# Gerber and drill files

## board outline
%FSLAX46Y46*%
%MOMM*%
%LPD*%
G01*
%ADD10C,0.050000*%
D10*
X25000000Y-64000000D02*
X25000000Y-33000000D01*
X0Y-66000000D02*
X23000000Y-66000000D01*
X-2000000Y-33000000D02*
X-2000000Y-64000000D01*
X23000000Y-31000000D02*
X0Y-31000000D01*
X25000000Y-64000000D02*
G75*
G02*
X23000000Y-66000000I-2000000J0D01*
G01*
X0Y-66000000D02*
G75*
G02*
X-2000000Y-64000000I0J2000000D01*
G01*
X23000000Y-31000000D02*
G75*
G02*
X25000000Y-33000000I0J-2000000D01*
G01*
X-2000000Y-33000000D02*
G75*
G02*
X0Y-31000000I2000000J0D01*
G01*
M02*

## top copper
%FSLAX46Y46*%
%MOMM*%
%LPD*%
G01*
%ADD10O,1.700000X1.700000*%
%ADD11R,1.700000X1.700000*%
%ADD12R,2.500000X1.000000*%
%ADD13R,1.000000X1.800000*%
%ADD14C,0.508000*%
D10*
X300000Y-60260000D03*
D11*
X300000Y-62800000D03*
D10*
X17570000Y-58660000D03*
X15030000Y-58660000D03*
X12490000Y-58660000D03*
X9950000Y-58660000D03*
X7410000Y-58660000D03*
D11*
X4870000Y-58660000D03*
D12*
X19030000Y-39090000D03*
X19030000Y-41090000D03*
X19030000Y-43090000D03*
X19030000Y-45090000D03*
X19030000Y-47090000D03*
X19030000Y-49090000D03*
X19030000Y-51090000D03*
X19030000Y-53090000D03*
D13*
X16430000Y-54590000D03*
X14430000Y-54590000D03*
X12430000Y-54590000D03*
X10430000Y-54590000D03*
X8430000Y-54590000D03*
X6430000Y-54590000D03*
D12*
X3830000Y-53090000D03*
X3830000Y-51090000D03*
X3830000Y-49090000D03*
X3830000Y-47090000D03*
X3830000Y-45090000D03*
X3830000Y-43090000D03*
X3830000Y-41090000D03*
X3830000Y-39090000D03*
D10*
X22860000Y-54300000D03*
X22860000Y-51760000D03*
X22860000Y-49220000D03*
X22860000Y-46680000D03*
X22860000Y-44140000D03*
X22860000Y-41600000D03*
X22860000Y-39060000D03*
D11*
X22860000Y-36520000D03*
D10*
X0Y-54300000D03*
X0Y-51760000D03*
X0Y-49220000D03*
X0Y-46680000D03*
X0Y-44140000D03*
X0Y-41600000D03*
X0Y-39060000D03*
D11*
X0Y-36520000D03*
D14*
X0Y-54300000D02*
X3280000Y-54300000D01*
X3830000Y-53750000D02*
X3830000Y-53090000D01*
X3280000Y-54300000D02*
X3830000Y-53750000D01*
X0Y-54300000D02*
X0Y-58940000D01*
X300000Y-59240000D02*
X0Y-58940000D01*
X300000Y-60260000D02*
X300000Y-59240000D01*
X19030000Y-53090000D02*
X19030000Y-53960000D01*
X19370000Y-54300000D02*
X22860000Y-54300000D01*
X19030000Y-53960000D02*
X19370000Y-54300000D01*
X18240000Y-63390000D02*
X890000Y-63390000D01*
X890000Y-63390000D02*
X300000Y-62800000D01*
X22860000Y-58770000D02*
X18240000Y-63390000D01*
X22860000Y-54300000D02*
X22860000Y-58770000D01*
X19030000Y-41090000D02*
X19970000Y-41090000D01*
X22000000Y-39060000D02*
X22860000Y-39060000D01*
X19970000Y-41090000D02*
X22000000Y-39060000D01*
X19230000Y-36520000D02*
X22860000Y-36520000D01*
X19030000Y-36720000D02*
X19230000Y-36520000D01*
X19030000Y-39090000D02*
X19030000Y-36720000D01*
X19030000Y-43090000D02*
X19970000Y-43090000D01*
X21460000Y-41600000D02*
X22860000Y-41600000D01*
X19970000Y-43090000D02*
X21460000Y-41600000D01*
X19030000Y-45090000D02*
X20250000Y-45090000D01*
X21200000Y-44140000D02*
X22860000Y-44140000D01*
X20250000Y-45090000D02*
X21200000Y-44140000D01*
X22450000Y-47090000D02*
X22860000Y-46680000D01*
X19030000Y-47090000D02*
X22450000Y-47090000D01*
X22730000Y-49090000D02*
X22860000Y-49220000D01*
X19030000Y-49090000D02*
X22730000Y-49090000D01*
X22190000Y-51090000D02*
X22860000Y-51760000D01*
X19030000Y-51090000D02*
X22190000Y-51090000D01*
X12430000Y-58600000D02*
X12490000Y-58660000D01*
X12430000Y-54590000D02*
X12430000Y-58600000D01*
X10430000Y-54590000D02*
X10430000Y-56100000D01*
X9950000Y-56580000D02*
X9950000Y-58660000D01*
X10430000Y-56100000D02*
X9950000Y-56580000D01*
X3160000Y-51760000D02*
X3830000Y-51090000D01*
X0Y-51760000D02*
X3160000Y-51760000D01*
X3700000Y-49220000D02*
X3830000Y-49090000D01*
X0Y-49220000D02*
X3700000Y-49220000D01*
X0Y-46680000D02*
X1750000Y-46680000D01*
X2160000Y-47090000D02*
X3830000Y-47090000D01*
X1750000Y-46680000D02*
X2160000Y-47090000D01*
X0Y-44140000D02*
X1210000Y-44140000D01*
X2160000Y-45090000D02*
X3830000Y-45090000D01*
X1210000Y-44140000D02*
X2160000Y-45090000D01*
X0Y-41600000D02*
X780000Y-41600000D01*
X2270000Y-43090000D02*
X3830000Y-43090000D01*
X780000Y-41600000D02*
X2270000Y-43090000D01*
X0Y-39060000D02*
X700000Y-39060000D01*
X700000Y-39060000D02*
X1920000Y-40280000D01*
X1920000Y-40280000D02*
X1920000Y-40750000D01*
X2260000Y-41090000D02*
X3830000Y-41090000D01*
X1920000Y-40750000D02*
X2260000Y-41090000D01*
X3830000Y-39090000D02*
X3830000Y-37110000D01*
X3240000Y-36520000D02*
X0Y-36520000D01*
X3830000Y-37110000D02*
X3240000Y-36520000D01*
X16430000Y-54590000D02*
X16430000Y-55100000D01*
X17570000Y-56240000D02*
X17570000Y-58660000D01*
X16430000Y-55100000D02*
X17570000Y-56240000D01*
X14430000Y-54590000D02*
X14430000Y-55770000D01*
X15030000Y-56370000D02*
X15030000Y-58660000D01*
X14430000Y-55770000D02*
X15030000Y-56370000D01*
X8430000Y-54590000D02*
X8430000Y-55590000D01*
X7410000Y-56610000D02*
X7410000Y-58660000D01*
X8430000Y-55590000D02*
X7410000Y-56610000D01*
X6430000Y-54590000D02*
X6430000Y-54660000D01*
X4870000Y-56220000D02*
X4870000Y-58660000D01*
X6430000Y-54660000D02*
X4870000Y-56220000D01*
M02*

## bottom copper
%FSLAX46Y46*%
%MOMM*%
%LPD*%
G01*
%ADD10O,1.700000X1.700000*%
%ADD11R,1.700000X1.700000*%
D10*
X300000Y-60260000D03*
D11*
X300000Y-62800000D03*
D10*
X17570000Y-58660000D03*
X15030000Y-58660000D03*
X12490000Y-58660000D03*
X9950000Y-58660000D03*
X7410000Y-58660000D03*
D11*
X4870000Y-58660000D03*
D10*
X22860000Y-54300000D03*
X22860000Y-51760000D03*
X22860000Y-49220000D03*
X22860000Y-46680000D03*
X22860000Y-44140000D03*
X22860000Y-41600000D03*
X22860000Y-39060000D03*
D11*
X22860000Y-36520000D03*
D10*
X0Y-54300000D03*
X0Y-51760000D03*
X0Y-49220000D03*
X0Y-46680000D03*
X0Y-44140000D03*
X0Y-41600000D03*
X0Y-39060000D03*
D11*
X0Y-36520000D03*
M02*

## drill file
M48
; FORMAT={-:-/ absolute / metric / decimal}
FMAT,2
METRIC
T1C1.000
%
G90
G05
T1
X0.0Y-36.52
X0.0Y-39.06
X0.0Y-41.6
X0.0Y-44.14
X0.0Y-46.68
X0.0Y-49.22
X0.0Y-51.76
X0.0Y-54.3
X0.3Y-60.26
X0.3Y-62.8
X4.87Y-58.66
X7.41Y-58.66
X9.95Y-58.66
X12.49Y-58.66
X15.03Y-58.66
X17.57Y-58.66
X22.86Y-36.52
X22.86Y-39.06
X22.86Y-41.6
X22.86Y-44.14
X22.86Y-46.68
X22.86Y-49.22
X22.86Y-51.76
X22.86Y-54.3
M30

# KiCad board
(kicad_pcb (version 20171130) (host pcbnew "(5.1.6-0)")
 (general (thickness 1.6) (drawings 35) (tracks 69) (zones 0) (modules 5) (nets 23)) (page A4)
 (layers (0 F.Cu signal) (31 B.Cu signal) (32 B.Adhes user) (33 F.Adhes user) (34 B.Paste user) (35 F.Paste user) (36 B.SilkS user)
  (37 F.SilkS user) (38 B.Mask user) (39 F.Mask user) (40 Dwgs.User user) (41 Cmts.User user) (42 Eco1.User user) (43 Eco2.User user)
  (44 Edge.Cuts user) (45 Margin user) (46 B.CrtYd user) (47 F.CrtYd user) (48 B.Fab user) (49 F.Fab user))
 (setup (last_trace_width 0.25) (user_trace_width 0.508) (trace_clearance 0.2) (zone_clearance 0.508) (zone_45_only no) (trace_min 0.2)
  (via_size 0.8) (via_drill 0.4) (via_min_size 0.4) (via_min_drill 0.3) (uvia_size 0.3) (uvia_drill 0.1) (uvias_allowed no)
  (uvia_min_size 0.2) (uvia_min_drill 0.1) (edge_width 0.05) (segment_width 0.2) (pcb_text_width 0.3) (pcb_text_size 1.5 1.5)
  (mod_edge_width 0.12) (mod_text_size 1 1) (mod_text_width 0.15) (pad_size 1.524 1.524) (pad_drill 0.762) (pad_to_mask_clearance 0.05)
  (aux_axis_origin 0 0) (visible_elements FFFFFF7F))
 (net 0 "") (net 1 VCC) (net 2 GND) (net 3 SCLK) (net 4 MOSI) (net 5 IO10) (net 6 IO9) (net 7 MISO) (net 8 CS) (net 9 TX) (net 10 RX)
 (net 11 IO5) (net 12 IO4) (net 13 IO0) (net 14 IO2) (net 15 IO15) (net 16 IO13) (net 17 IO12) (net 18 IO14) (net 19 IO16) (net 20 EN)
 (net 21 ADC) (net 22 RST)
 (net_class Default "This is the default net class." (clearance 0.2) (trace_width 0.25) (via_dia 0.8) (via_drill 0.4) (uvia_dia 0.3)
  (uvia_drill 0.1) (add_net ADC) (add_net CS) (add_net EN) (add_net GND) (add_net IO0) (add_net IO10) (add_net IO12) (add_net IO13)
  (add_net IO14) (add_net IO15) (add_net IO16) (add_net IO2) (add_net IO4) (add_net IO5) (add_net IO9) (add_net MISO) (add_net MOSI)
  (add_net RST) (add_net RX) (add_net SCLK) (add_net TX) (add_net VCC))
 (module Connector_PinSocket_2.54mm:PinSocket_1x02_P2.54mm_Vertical (layer F.Cu) (at 0.3 62.8 180)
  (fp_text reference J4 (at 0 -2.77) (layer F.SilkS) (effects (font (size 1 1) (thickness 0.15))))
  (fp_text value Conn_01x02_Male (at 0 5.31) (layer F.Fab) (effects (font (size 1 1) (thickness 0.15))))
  (pad 2 thru_hole oval (at 0 2.54 180) (size 1.7 1.7) (drill 1) (layers *.Cu *.Mask) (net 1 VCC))
  (pad 1 thru_hole rect (at 0 0 180) (size 1.7 1.7) (drill 1) (layers *.Cu *.Mask) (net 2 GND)))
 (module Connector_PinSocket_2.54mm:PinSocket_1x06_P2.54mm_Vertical (layer F.Cu) (at 4.87 58.66 90)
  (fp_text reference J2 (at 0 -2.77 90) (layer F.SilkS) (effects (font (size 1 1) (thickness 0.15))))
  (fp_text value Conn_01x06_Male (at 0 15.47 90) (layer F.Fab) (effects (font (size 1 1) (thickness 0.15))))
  (pad 6 thru_hole oval (at 0 12.7 90) (size 1.7 1.7) (drill 1) (layers *.Cu *.Mask) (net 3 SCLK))
  (pad 5 thru_hole oval (at 0 10.16 90) (size 1.7 1.7) (drill 1) (layers *.Cu *.Mask) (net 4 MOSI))
  (pad 4 thru_hole oval (at 0 7.62 90) (size 1.7 1.7) (drill 1) (layers *.Cu *.Mask) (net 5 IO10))
  (pad 3 thru_hole oval (at 0 5.08 90) (size 1.7 1.7) (drill 1) (layers *.Cu *.Mask) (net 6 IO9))
  (pad 2 thru_hole oval (at 0 2.54 90) (size 1.7 1.7) (drill 1) (layers *.Cu *.Mask) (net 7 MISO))
  (pad 1 thru_hole rect (at 0 0 90) (size 1.7 1.7) (drill 1) (layers *.Cu *.Mask) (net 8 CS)))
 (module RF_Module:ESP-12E (layer F.Cu) (at 11.43 42.59)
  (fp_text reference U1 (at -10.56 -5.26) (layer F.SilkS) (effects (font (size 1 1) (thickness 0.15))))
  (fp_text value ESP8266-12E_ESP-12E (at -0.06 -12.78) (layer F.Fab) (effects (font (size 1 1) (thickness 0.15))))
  (pad 22 smd rect (at 7.6 -3.5) (size 2.5 1) (layers F.Cu F.Paste F.Mask) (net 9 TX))
  (pad 21 smd rect (at 7.6 -1.5) (size 2.5 1) (layers F.Cu F.Paste F.Mask) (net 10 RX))
  (pad 20 smd rect (at 7.6 0.5) (size 2.5 1) (layers F.Cu F.Paste F.Mask) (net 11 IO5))
  (pad 19 smd rect (at 7.6 2.5) (size 2.5 1) (layers F.Cu F.Paste F.Mask) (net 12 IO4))
  (pad 18 smd rect (at 7.6 4.5) (size 2.5 1) (layers F.Cu F.Paste F.Mask) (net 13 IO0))
  (pad 17 smd rect (at 7.6 6.5) (size 2.5 1) (layers F.Cu F.Paste F.Mask) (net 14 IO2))
  (pad 16 smd rect (at 7.6 8.5) (size 2.5 1) (layers F.Cu F.Paste F.Mask) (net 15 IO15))
  (pad 15 smd rect (at 7.6 10.5) (size 2.5 1) (layers F.Cu F.Paste F.Mask) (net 2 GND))
  (pad 14 smd rect (at 5 12) (size 1 1.8) (layers F.Cu F.Paste F.Mask) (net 3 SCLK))
  (pad 13 smd rect (at 3 12) (size 1 1.8) (layers F.Cu F.Paste F.Mask) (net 4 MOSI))
  (pad 12 smd rect (at 1 12) (size 1 1.8) (layers F.Cu F.Paste F.Mask) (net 5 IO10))
  (pad 11 smd rect (at -1 12) (size 1 1.8) (layers F.Cu F.Paste F.Mask) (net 6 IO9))
  (pad 10 smd rect (at -3 12) (size 1 1.8) (layers F.Cu F.Paste F.Mask) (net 7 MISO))
  (pad 9 smd rect (at -5 12) (size 1 1.8) (layers F.Cu F.Paste F.Mask) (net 8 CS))
  (pad 8 smd rect (at -7.6 10.5) (size 2.5 1) (layers F.Cu F.Paste F.Mask) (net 1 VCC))
  (pad 7 smd rect (at -7.6 8.5) (size 2.5 1) (layers F.Cu F.Paste F.Mask) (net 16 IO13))
  (pad 6 smd rect (at -7.6 6.5) (size 2.5 1) (layers F.Cu F.Paste F.Mask) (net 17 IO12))
  (pad 5 smd rect (at -7.6 4.5) (size 2.5 1) (layers F.Cu F.Paste F.Mask) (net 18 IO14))
  (pad 4 smd rect (at -7.6 2.5) (size 2.5 1) (layers F.Cu F.Paste F.Mask) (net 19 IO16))
  (pad 3 smd rect (at -7.6 0.5) (size 2.5 1) (layers F.Cu F.Paste F.Mask) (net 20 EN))
  (pad 2 smd rect (at -7.6 -1.5) (size 2.5 1) (layers F.Cu F.Paste F.Mask) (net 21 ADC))
  (pad 1 smd rect (at -7.6 -3.5) (size 2.5 1) (layers F.Cu F.Paste F.Mask) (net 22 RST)))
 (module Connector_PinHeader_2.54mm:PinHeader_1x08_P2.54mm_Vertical (layer F.Cu) (at 22.86 36.52)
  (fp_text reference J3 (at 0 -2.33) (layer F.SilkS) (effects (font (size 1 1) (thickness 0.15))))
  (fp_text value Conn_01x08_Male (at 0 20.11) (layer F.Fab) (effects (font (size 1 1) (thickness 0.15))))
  (pad 8 thru_hole oval (at 0 17.78) (size 1.7 1.7) (drill 1) (layers *.Cu *.Mask) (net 2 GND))
  (pad 7 thru_hole oval (at 0 15.24) (size 1.7 1.7) (drill 1) (layers *.Cu *.Mask) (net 15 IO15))
  (pad 6 thru_hole oval (at 0 12.7) (size 1.7 1.7) (drill 1) (layers *.Cu *.Mask) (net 14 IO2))
  (pad 5 thru_hole oval (at 0 10.16) (size 1.7 1.7) (drill 1) (layers *.Cu *.Mask) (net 13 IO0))
  (pad 4 thru_hole oval (at 0 7.62) (size 1.7 1.7) (drill 1) (layers *.Cu *.Mask) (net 12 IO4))
  (pad 3 thru_hole oval (at 0 5.08) (size 1.7 1.7) (drill 1) (layers *.Cu *.Mask) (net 11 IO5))
  (pad 2 thru_hole oval (at 0 2.54) (size 1.7 1.7) (drill 1) (layers *.Cu *.Mask) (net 10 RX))
  (pad 1 thru_hole rect (at 0 0) (size 1.7 1.7) (drill 1) (layers *.Cu *.Mask) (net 9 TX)))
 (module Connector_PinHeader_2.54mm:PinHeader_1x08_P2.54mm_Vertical (layer F.Cu) (at 0 36.52)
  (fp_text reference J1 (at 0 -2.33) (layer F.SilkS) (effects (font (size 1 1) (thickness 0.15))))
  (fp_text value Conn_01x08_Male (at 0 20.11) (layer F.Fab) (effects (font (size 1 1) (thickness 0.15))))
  (pad 8 thru_hole oval (at 0 17.78) (size 1.7 1.7) (drill 1) (layers *.Cu *.Mask) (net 1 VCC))
  (pad 7 thru_hole oval (at 0 15.24) (size 1.7 1.7) (drill 1) (layers *.Cu *.Mask) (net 16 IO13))
  (pad 6 thru_hole oval (at 0 12.7) (size 1.7 1.7) (drill 1) (layers *.Cu *.Mask) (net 17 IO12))
  (pad 5 thru_hole oval (at 0 10.16) (size 1.7 1.7) (drill 1) (layers *.Cu *.Mask) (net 18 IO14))
  (pad 4 thru_hole oval (at 0 7.62) (size 1.7 1.7) (drill 1) (layers *.Cu *.Mask) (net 19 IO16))
  (pad 3 thru_hole oval (at 0 5.08) (size 1.7 1.7) (drill 1) (layers *.Cu *.Mask) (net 20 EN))
  (pad 2 thru_hole oval (at 0 2.54) (size 1.7 1.7) (drill 1) (layers *.Cu *.Mask) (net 21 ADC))
  (pad 1 thru_hole rect (at 0 0) (size 1.7 1.7) (drill 1) (layers *.Cu *.Mask) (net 22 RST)))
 (gr_line (start 25 64) (end 25 33) (layer Edge.Cuts) (width 0.05))
 (gr_line (start 0 66) (end 23 66) (layer Edge.Cuts) (width 0.05))
 (gr_line (start -2 33) (end -2 64) (layer Edge.Cuts) (width 0.05))
 (gr_line (start 23 31) (end 0 31) (layer Edge.Cuts) (width 0.05))
 (gr_arc (start 23 64) (end 23 66) (angle -90) (layer Edge.Cuts) (width 0.05))
 (gr_arc (start 0 64) (end -2 64) (angle -90) (layer Edge.Cuts) (width 0.05))
 (gr_arc (start 23 33) (end 25 33) (angle -90) (layer Edge.Cuts) (width 0.05))
 (gr_arc (start 0 33) (end 0 31) (angle -90) (layer Edge.Cuts) (width 0.05))
 (segment (start 0 54.3) (end 3.28 54.3) (width 0.508) (layer F.Cu) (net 1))
 (segment (start 3.83 53.75) (end 3.83 53.09) (width 0.508) (layer F.Cu) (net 1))
 (segment (start 3.28 54.3) (end 3.83 53.75) (width 0.508) (layer F.Cu) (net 1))
 (segment (start 0 54.3) (end 0 58.94) (width 0.508) (layer F.Cu) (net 1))
 (segment (start 0.3 59.24) (end 0 58.94) (width 0.508) (layer F.Cu) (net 1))
 (segment (start 0.3 60.26) (end 0.3 59.24) (width 0.508) (layer F.Cu) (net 1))
 (segment (start 19.03 53.09) (end 19.03 53.96) (width 0.508) (layer F.Cu) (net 2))
 (segment (start 19.37 54.3) (end 22.86 54.3) (width 0.508) (layer F.Cu) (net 2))
 (segment (start 19.03 53.96) (end 19.37 54.3) (width 0.508) (layer F.Cu) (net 2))
 (segment (start 18.24 63.39) (end 0.89 63.39) (width 0.508) (layer F.Cu) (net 2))
 (segment (start 0.89 63.39) (end 0.3 62.8) (width 0.508) (layer F.Cu) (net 2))
 (segment (start 22.86 58.77) (end 18.24 63.39) (width 0.508) (layer F.Cu) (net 2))
 (segment (start 22.86 54.3) (end 22.86 58.77) (width 0.508) (layer F.Cu) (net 2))
 (segment (start 19.03 41.09) (end 19.97 41.09) (width 0.508) (layer F.Cu) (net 10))
 (segment (start 22 39.06) (end 22.86 39.06) (width 0.508) (layer F.Cu) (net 10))
 (segment (start 19.97 41.09) (end 22 39.06) (width 0.508) (layer F.Cu) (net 10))
 (segment (start 19.23 36.52) (end 22.86 36.52) (width 0.508) (layer F.Cu) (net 9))
 (segment (start 19.03 36.72) (end 19.23 36.52) (width 0.508) (layer F.Cu) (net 9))
 (segment (start 19.03 39.09) (end 19.03 36.72) (width 0.508) (layer F.Cu) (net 9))
 (segment (start 19.03 43.09) (end 19.97 43.09) (width 0.508) (layer F.Cu) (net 11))
 (segment (start 21.46 41.6) (end 22.86 41.6) (width 0.508) (layer F.Cu) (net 11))
 (segment (start 19.97 43.09) (end 21.46 41.6) (width 0.508) (layer F.Cu) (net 11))
 (segment (start 19.03 45.09) (end 20.25 45.09) (width 0.508) (layer F.Cu) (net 12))
 (segment (start 21.2 44.14) (end 22.86 44.14) (width 0.508) (layer F.Cu) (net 12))
 (segment (start 20.25 45.09) (end 21.2 44.14) (width 0.508) (layer F.Cu) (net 12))
 (segment (start 22.45 47.09) (end 22.86 46.68) (width 0.508) (layer F.Cu) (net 13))
 (segment (start 19.03 47.09) (end 22.45 47.09) (width 0.508) (layer F.Cu) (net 13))
 (segment (start 22.73 49.09) (end 22.86 49.22) (width 0.508) (layer F.Cu) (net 14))
 (segment (start 19.03 49.09) (end 22.73 49.09) (width 0.508) (layer F.Cu) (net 14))
 (segment (start 22.19 51.09) (end 22.86 51.76) (width 0.508) (layer F.Cu) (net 15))
 (segment (start 19.03 51.09) (end 22.19 51.09) (width 0.508) (layer F.Cu) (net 15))
 (segment (start 12.43 58.6) (end 12.49 58.66) (width 0.508) (layer F.Cu) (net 5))
 (segment (start 12.43 54.59) (end 12.43 58.6) (width 0.508) (layer F.Cu) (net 5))
 (segment (start 10.43 54.59) (end 10.43 56.1) (width 0.508) (layer F.Cu) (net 6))
 (segment (start 9.95 56.58) (end 9.95 58.66) (width 0.508) (layer F.Cu) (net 6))
 (segment (start 10.43 56.1) (end 9.95 56.58) (width 0.508) (layer F.Cu) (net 6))
 (segment (start 3.16 51.76) (end 3.83 51.09) (width 0.508) (layer F.Cu) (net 16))
 (segment (start 0 51.76) (end 3.16 51.76) (width 0.508) (layer F.Cu) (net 16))
 (segment (start 3.7 49.22) (end 3.83 49.09) (width 0.508) (layer F.Cu) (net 17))
 (segment (start 0 49.22) (end 3.7 49.22) (width 0.508) (layer F.Cu) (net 17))
 (segment (start 0 46.68) (end 1.75 46.68) (width 0.508) (layer F.Cu) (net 18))
 (segment (start 2.16 47.09) (end 3.83 47.09) (width 0.508) (layer F.Cu) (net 18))
 (segment (start 1.75 46.68) (end 2.16 47.09) (width 0.508) (layer F.Cu) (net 18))
 (segment (start 0 44.14) (end 1.21 44.14) (width 0.508) (layer F.Cu) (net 19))
 (segment (start 2.16 45.09) (end 3.83 45.09) (width 0.508) (layer F.Cu) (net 19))
 (segment (start 1.21 44.14) (end 2.16 45.09) (width 0.508) (layer F.Cu) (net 19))
 (segment (start 0 41.6) (end 0.78 41.6) (width 0.508) (layer F.Cu) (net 20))
 (segment (start 2.27 43.09) (end 3.83 43.09) (width 0.508) (layer F.Cu) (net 20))
 (segment (start 0.78 41.6) (end 2.27 43.09) (width 0.508) (layer F.Cu) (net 20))
 (segment (start 0 39.06) (end 0.7 39.06) (width 0.508) (layer F.Cu) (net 21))
 (segment (start 0.7 39.06) (end 1.92 40.28) (width 0.508) (layer F.Cu) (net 21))
 (segment (start 1.92 40.28) (end 1.92 40.75) (width 0.508) (layer F.Cu) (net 21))
 (segment (start 2.26 41.09) (end 3.83 41.09) (width 0.508) (layer F.Cu) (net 21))
 (segment (start 1.92 40.75) (end 2.26 41.09) (width 0.508) (layer F.Cu) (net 21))
 (segment (start 3.83 39.09) (end 3.83 37.11) (width 0.508) (layer F.Cu) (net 22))
 (segment (start 3.24 36.52) (end 0 36.52) (width 0.508) (layer F.Cu) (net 22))
 (segment (start 3.83 37.11) (end 3.24 36.52) (width 0.508) (layer F.Cu) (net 22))
 (segment (start 16.43 54.59) (end 16.43 55.1) (width 0.508) (layer F.Cu) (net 3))
 (segment (start 17.57 56.24) (end 17.57 58.66) (width 0.508) (layer F.Cu) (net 3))
 (segment (start 16.43 55.1) (end 17.57 56.24) (width 0.508) (layer F.Cu) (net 3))
 (segment (start 14.43 54.59) (end 14.43 55.77) (width 0.508) (layer F.Cu) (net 4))
 (segment (start 15.03 56.37) (end 15.03 58.66) (width 0.508) (layer F.Cu) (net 4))
 (segment (start 14.43 55.77) (end 15.03 56.37) (width 0.508) (layer F.Cu) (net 4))
 (segment (start 8.43 54.59) (end 8.43 55.59) (width 0.508) (layer F.Cu) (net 7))
 (segment (start 7.41 56.61) (end 7.41 58.66) (width 0.508) (layer F.Cu) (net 7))
 (segment (start 8.43 55.59) (end 7.41 56.61) (width 0.508) (layer F.Cu) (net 7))
 (segment (start 6.43 54.59) (end 6.43 54.66) (width 0.508) (layer F.Cu) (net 8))
 (segment (start 4.87 56.22) (end 4.87 58.66) (width 0.508) (layer F.Cu) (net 8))
 (segment (start 6.43 54.66) (end 4.87 56.22) (width 0.508) (layer F.Cu) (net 8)))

